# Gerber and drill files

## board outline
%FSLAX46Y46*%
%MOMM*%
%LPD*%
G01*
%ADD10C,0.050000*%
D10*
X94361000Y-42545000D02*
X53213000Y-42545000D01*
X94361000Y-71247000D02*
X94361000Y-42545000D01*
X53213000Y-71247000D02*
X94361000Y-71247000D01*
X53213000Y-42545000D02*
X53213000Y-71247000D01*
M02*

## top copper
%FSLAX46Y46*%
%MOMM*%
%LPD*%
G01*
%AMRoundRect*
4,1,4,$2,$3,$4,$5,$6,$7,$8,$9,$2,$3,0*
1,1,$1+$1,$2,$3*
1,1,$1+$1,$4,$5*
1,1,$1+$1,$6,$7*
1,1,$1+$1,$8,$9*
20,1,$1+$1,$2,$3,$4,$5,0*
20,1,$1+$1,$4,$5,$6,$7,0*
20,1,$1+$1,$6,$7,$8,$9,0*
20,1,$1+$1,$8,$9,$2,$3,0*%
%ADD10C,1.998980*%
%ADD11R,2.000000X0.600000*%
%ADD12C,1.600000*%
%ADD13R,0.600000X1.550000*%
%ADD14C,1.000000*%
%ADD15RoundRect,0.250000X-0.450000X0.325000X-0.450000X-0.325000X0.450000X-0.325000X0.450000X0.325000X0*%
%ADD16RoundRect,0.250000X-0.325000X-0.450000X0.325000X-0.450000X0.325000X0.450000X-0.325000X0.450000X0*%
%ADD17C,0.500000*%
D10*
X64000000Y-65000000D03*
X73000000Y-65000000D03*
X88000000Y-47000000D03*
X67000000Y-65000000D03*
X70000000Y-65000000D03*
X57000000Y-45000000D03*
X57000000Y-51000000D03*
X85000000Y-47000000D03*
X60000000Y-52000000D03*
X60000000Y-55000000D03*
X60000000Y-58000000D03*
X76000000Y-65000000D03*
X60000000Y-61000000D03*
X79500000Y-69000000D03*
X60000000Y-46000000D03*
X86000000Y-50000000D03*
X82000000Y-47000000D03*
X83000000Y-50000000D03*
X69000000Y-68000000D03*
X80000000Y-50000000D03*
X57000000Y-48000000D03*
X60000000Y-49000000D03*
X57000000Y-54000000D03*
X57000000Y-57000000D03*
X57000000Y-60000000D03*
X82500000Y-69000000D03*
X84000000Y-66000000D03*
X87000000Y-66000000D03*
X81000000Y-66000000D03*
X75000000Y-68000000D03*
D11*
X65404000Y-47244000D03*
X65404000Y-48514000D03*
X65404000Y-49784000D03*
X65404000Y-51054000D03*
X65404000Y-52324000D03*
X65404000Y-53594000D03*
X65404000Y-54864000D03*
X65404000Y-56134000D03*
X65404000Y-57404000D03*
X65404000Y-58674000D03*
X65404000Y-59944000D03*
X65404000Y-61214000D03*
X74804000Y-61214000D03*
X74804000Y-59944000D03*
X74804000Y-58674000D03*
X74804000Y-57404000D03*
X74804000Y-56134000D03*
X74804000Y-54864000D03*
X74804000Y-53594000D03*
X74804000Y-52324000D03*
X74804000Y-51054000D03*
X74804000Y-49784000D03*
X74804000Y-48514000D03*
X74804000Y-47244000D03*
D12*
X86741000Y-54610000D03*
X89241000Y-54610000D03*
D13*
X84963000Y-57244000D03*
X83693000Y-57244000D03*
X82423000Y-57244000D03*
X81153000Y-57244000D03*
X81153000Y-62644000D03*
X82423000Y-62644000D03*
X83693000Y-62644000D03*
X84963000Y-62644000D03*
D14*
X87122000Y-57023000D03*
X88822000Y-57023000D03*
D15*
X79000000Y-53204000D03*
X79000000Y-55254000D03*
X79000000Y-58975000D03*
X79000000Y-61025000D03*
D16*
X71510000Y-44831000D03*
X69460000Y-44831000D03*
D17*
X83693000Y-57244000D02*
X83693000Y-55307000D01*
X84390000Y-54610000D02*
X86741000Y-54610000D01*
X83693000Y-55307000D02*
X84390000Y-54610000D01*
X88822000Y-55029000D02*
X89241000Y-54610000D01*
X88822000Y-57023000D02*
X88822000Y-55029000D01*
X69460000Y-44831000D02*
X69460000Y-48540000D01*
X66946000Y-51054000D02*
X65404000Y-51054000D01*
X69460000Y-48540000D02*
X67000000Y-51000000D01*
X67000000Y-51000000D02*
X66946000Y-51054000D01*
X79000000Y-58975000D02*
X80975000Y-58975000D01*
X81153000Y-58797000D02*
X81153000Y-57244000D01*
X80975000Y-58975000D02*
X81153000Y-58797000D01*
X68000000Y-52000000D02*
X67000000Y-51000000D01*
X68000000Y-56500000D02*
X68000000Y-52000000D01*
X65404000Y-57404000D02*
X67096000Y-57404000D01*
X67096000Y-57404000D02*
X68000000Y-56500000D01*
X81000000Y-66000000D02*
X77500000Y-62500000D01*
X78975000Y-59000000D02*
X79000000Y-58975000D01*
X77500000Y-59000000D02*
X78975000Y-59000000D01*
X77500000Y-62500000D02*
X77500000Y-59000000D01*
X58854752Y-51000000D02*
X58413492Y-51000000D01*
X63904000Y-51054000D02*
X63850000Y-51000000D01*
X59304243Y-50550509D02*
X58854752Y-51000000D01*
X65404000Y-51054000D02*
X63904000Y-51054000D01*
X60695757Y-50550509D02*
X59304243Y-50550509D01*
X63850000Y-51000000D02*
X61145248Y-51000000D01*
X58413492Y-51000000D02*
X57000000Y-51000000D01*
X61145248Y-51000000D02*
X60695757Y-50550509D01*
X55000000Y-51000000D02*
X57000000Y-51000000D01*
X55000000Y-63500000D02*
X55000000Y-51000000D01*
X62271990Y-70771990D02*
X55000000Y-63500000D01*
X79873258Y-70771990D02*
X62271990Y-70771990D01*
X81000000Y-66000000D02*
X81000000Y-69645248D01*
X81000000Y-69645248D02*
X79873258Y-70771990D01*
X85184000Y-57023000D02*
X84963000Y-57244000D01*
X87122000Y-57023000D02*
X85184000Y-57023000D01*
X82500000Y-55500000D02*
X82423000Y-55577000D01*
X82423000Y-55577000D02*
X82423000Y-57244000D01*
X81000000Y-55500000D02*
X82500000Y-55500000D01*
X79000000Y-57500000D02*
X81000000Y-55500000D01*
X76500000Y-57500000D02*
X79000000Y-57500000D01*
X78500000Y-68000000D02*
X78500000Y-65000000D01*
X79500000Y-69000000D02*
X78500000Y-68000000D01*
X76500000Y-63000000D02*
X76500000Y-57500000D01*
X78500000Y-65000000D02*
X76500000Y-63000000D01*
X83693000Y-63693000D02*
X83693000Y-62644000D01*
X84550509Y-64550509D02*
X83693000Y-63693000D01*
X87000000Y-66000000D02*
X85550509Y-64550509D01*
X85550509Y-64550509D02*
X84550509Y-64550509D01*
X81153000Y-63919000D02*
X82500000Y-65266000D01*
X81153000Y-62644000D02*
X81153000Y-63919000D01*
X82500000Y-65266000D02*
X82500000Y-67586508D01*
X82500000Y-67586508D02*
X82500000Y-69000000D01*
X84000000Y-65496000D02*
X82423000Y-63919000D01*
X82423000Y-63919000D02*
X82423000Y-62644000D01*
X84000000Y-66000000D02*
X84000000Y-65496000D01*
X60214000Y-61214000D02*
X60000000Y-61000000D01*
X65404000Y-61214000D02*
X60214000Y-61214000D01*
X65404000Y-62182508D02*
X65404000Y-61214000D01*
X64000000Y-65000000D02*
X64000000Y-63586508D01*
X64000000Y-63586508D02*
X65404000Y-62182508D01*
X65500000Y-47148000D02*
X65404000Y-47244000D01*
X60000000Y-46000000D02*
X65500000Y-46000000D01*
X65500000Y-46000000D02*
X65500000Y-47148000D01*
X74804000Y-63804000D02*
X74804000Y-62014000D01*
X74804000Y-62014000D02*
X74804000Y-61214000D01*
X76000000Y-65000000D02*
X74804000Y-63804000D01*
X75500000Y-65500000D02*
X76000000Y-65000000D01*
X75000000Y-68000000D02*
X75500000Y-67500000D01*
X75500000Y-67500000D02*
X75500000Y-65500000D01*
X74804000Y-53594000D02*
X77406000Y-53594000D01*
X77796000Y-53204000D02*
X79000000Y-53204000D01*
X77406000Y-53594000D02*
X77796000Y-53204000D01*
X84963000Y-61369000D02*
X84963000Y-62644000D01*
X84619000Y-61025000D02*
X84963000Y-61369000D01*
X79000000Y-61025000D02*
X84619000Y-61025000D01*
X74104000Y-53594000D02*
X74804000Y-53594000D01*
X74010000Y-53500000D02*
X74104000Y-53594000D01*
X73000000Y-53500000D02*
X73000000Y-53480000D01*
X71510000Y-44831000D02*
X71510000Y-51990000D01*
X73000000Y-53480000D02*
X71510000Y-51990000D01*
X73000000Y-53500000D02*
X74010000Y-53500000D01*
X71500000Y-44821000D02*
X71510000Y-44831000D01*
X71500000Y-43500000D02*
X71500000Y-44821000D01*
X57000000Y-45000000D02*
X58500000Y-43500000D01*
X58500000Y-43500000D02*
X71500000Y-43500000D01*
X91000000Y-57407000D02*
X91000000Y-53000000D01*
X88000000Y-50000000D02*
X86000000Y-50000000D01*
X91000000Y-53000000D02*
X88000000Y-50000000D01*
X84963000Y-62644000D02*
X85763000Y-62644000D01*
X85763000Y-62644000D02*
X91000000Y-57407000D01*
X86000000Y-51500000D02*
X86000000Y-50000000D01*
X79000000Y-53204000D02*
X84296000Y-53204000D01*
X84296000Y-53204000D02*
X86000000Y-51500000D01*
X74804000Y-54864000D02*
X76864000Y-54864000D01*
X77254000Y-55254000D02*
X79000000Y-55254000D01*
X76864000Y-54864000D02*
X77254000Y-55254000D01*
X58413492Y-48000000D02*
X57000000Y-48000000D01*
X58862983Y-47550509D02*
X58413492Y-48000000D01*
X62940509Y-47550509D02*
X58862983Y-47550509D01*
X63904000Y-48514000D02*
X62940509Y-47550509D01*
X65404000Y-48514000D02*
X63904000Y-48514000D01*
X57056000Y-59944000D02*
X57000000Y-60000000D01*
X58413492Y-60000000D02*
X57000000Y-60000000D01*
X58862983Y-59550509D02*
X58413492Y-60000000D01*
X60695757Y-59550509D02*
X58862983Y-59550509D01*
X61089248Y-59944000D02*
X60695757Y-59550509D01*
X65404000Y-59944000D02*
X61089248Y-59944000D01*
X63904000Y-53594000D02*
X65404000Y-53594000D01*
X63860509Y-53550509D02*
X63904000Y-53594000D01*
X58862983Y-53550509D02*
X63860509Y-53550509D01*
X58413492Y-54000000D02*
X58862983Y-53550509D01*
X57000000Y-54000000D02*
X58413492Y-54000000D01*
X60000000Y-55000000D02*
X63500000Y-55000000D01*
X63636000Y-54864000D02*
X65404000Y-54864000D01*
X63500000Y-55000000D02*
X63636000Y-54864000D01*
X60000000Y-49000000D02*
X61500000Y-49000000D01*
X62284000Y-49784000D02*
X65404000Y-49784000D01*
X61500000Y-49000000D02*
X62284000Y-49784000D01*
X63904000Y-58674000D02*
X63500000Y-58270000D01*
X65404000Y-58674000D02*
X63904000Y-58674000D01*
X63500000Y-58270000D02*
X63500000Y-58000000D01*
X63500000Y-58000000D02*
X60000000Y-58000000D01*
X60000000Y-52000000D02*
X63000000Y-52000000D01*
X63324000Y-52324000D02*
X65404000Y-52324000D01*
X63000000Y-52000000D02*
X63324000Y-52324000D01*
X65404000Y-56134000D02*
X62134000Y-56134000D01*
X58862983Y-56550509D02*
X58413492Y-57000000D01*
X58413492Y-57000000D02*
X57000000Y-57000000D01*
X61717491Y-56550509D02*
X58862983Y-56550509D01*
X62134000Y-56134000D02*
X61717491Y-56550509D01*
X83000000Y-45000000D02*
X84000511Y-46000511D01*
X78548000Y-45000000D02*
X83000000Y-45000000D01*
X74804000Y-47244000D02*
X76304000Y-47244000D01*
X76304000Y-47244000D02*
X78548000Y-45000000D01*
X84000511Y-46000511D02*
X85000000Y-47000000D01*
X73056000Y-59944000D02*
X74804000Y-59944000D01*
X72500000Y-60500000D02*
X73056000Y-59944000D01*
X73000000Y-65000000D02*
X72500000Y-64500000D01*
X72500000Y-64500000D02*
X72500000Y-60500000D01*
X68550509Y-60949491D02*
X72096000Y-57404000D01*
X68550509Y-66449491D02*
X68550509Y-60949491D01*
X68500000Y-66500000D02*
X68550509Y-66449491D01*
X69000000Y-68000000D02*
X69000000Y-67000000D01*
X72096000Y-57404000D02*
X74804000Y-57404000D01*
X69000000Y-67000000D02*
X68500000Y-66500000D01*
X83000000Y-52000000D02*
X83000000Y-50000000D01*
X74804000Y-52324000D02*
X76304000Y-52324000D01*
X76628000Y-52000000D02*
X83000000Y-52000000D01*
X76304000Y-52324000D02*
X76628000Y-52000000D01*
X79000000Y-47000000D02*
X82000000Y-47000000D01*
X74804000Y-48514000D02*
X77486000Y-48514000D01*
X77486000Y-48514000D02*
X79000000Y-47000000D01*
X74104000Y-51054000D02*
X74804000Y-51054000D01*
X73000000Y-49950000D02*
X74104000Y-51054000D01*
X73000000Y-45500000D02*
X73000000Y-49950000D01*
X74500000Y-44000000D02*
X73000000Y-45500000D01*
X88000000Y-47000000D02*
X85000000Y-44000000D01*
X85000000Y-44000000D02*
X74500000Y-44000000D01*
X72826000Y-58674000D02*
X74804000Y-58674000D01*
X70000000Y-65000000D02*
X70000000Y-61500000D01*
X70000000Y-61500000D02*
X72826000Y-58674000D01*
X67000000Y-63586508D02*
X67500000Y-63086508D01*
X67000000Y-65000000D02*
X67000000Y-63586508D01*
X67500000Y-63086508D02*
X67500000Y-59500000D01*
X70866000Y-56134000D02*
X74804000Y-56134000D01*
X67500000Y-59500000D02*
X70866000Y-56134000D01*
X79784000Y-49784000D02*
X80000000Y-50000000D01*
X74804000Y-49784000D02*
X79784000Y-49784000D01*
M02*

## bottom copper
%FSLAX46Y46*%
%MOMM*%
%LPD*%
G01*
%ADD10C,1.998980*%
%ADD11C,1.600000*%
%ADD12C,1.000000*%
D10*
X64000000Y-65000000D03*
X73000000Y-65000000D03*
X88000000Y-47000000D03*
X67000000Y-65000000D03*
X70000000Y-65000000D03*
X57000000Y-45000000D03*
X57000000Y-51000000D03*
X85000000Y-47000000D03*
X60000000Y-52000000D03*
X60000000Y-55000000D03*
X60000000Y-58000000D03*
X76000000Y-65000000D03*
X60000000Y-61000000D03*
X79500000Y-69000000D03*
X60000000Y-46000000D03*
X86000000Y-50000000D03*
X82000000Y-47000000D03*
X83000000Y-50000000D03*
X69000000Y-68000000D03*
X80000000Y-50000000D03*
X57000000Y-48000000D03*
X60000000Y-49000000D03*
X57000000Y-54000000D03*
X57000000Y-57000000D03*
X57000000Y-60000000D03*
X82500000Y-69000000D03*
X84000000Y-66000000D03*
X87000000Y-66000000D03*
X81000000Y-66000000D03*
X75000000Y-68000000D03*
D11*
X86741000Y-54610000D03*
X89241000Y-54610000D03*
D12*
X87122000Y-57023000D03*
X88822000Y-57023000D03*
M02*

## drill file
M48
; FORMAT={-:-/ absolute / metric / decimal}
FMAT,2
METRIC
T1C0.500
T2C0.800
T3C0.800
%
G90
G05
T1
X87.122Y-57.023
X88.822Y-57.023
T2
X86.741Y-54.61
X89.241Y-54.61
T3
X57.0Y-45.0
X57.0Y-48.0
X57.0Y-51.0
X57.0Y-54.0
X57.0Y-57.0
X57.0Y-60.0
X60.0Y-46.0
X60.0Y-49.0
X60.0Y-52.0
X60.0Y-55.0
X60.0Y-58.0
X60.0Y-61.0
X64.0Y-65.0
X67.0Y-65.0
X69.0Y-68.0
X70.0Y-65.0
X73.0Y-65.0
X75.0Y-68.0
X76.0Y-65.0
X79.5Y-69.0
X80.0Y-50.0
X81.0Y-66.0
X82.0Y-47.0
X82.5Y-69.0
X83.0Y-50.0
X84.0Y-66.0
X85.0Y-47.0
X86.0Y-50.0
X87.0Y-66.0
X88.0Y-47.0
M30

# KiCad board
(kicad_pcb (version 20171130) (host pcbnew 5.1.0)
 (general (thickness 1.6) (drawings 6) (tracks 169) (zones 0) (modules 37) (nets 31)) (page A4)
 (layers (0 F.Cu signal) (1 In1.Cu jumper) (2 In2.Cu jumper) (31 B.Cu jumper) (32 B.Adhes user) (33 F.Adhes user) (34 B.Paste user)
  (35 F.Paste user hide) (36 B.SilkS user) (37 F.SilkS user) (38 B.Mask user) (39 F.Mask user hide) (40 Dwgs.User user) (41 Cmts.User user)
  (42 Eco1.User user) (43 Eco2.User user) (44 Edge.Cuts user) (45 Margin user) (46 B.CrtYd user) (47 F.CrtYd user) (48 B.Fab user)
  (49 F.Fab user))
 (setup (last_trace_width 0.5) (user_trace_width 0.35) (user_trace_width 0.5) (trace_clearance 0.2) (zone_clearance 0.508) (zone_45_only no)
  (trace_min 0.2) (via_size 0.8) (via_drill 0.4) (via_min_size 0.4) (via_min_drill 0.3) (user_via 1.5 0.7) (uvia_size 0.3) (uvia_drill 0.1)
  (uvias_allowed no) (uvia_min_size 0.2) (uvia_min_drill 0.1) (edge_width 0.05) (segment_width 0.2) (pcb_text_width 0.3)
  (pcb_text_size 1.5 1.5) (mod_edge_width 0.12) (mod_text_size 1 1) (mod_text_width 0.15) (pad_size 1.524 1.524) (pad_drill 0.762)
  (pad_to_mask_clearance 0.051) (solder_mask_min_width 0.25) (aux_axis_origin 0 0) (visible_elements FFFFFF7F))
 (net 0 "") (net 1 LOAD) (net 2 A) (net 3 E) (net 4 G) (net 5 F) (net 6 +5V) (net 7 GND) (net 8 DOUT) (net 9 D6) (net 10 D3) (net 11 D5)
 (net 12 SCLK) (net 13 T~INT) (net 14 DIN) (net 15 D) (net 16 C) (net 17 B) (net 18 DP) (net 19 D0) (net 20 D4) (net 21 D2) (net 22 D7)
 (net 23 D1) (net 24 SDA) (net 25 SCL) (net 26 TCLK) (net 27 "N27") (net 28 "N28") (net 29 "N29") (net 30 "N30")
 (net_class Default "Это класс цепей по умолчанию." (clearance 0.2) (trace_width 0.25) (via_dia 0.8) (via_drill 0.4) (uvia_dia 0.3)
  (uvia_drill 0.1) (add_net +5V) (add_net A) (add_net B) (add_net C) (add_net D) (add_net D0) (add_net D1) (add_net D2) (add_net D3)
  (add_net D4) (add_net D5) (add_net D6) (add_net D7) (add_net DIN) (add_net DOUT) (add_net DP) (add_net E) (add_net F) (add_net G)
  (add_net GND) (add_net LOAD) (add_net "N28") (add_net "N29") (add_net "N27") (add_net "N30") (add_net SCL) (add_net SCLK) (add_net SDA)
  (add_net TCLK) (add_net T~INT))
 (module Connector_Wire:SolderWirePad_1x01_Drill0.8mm (layer F.Cu) (at 64 65)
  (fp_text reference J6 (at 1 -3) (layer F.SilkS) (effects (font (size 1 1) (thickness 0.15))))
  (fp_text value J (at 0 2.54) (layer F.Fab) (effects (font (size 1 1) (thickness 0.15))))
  (pad 1 thru_hole circle (at 0 0) (size 1.99898 1.99898) (drill 0.8001) (layers *.Cu *.Mask) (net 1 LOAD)))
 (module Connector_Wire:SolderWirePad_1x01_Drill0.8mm (layer F.Cu) (at 73 65)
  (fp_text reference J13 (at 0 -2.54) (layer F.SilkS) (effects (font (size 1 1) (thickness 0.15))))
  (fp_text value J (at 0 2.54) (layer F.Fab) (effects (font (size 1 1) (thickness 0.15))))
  (pad 1 thru_hole circle (at 0 0) (size 1.99898 1.99898) (drill 0.8001) (layers *.Cu *.Mask) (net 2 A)))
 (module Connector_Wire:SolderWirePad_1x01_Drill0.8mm (layer F.Cu) (at 88 47)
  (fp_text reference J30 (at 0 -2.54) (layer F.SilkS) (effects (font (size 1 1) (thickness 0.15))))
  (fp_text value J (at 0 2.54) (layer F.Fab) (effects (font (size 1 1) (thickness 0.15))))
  (pad 1 thru_hole circle (at 0 0) (size 1.99898 1.99898) (drill 0.8001) (layers *.Cu *.Mask) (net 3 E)))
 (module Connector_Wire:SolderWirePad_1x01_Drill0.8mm (layer F.Cu) (at 67 65)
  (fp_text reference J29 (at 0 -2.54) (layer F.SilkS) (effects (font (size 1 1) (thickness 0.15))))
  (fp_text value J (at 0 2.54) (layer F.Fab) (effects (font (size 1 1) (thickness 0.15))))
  (pad 1 thru_hole circle (at 0 0) (size 1.99898 1.99898) (drill 0.8001) (layers *.Cu *.Mask) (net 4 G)))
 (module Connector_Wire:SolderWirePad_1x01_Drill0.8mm (layer F.Cu) (at 70 65)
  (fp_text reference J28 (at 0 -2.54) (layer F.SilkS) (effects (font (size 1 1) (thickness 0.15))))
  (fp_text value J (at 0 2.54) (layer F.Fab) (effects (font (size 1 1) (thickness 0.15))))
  (pad 1 thru_hole circle (at 0 0) (size 1.99898 1.99898) (drill 0.8001) (layers *.Cu *.Mask) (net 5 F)))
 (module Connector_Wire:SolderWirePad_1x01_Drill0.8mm (layer F.Cu) (at 57 45)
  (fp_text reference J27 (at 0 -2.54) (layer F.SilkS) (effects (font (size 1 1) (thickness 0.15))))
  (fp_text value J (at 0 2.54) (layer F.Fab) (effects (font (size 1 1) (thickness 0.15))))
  (pad 1 thru_hole circle (at 0 0) (size 1.99898 1.99898) (drill 0.8001) (layers *.Cu *.Mask) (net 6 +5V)))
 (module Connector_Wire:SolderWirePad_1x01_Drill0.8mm (layer F.Cu) (at 57 51)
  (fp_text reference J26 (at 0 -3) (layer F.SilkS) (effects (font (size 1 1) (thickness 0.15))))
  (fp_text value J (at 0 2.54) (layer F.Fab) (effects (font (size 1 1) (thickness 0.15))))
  (pad 1 thru_hole circle (at 0 0) (size 1.99898 1.99898) (drill 0.8001) (layers *.Cu *.Mask) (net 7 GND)))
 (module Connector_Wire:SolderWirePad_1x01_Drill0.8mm (layer F.Cu) (at 85 47)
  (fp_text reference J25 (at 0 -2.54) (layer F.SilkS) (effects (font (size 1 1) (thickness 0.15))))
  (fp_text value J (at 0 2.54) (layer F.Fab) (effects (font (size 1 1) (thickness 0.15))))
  (pad 1 thru_hole circle (at 0 0) (size 1.99898 1.99898) (drill 0.8001) (layers *.Cu *.Mask) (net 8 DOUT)))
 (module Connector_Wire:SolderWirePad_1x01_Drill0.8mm (layer F.Cu) (at 60 52)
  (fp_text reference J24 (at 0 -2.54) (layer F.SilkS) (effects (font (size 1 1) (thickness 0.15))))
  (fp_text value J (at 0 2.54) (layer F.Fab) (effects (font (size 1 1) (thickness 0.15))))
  (pad 1 thru_hole circle (at 0 0) (size 1.99898 1.99898) (drill 0.8001) (layers *.Cu *.Mask) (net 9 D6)))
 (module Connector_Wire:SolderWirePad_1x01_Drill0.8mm (layer F.Cu) (at 60 55)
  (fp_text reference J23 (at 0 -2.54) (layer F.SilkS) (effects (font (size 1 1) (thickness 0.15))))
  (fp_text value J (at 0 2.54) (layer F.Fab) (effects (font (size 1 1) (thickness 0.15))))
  (pad 1 thru_hole circle (at 0 0) (size 1.99898 1.99898) (drill 0.8001) (layers *.Cu *.Mask) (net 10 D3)))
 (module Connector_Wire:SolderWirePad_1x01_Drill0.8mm (layer F.Cu) (at 60 58)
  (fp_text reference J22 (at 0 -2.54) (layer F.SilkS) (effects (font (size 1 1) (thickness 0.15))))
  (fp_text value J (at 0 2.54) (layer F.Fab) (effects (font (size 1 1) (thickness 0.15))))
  (pad 1 thru_hole circle (at 0 0) (size 1.99898 1.99898) (drill 0.8001) (layers *.Cu *.Mask) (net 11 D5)))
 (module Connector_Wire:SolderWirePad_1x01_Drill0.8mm (layer F.Cu) (at 76 65)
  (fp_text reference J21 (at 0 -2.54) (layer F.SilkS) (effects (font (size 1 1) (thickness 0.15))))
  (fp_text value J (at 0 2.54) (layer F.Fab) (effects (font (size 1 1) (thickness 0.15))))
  (pad 1 thru_hole circle (at 0 0) (size 1.99898 1.99898) (drill 0.8001) (layers *.Cu *.Mask) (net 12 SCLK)))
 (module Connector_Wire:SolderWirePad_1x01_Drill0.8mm (layer F.Cu) (at 60 61)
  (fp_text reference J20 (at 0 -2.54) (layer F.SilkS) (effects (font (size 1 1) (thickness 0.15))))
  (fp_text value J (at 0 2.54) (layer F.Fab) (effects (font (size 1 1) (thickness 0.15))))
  (pad 1 thru_hole circle (at 0 0) (size 1.99898 1.99898) (drill 0.8001) (layers *.Cu *.Mask) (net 1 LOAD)))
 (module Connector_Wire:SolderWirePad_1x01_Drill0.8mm (layer F.Cu) (at 79.5 69)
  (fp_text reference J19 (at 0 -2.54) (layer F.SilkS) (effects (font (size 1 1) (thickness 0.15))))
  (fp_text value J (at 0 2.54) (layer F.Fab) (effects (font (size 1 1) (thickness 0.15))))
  (pad 1 thru_hole circle (at 0 0) (size 1.99898 1.99898) (drill 0.8001) (layers *.Cu *.Mask) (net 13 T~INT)))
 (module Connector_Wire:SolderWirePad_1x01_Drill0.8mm (layer F.Cu) (at 60 46)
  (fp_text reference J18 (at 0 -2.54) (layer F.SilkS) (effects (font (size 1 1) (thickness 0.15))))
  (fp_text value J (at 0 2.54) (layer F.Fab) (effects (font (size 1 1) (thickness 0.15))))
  (pad 1 thru_hole circle (at 0 0) (size 1.99898 1.99898) (drill 0.8001) (layers *.Cu *.Mask) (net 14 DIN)))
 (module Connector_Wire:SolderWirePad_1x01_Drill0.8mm (layer F.Cu) (at 86 50)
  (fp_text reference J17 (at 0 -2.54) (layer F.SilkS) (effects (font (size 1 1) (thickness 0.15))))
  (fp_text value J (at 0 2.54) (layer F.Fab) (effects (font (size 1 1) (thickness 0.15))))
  (pad 1 thru_hole circle (at 0 0) (size 1.99898 1.99898) (drill 0.8001) (layers *.Cu *.Mask) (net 6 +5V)))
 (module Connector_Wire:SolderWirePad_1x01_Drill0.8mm (layer F.Cu) (at 82 47)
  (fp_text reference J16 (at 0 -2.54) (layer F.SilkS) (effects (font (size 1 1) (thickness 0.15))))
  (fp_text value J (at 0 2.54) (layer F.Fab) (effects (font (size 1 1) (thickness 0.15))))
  (pad 1 thru_hole circle (at 0 0) (size 1.99898 1.99898) (drill 0.8001) (layers *.Cu *.Mask) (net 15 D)))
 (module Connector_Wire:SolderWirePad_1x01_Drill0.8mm (layer F.Cu) (at 83 50)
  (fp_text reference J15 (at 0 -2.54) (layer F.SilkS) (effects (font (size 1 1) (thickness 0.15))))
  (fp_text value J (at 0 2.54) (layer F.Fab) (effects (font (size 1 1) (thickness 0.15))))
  (pad 1 thru_hole circle (at 0 0) (size 1.99898 1.99898) (drill 0.8001) (layers *.Cu *.Mask) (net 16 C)))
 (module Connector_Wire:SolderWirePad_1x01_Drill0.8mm (layer F.Cu) (at 69 68)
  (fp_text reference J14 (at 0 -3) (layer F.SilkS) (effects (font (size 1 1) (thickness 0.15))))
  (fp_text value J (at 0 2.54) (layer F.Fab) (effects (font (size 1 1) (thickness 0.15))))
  (pad 1 thru_hole circle (at 0 0) (size 1.99898 1.99898) (drill 0.8001) (layers *.Cu *.Mask) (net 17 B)))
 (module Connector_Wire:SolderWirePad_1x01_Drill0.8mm (layer F.Cu) (at 80 50)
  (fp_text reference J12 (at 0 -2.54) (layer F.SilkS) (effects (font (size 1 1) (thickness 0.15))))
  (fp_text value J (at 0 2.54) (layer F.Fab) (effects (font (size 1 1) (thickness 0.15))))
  (pad 1 thru_hole circle (at 0 0) (size 1.99898 1.99898) (drill 0.8001) (layers *.Cu *.Mask) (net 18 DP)))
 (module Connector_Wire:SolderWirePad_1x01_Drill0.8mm (layer F.Cu) (at 57 48)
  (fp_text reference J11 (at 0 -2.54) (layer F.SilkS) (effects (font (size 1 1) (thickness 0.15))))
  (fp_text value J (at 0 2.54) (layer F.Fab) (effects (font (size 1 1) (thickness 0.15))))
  (pad 1 thru_hole circle (at 0 0) (size 1.99898 1.99898) (drill 0.8001) (layers *.Cu *.Mask) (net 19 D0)))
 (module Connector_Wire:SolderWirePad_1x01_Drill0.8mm (layer F.Cu) (at 60 49)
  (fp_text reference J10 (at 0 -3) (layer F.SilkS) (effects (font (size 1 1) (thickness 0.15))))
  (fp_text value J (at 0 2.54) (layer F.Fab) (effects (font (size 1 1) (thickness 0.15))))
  (pad 1 thru_hole circle (at 0 0) (size 1.99898 1.99898) (drill 0.8001) (layers *.Cu *.Mask) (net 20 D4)))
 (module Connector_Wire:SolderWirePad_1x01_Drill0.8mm (layer F.Cu) (at 57 54)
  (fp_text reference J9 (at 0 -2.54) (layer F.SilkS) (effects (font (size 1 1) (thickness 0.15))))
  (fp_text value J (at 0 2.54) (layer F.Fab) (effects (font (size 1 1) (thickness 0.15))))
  (pad 1 thru_hole circle (at 0 0) (size 1.99898 1.99898) (drill 0.8001) (layers *.Cu *.Mask) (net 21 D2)))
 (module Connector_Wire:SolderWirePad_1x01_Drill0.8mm (layer F.Cu) (at 57 57)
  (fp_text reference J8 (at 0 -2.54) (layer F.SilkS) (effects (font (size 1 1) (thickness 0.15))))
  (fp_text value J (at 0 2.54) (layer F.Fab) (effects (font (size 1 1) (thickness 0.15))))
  (pad 1 thru_hole circle (at 0 0) (size 1.99898 1.99898) (drill 0.8001) (layers *.Cu *.Mask) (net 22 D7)))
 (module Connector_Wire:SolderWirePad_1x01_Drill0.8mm (layer F.Cu) (at 57 60)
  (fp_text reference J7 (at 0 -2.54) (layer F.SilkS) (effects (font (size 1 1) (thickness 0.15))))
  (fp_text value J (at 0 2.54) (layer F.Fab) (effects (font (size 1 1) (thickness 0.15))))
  (pad 1 thru_hole circle (at 0 0) (size 1.99898 1.99898) (drill 0.8001) (layers *.Cu *.Mask) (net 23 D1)))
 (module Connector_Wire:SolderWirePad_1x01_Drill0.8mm (layer F.Cu) (at 82.5 69)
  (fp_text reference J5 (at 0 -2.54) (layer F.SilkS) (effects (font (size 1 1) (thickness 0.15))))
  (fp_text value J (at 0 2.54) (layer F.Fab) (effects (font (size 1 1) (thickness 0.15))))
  (pad 1 thru_hole circle (at 0 0) (size 1.99898 1.99898) (drill 0.8001) (layers *.Cu *.Mask) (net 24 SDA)))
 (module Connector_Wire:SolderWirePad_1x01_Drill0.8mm (layer F.Cu) (at 84 66)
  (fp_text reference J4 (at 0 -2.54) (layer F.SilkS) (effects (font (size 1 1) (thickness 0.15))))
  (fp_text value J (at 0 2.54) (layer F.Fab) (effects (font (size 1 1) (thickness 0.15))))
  (pad 1 thru_hole circle (at 0 0) (size 1.99898 1.99898) (drill 0.8001) (layers *.Cu *.Mask) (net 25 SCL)))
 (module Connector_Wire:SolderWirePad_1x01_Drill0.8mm (layer F.Cu) (at 87 66)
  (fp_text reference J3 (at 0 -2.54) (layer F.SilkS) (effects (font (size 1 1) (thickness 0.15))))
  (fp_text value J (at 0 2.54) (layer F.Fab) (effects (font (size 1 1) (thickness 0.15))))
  (pad 1 thru_hole circle (at 0 0) (size 1.99898 1.99898) (drill 0.8001) (layers *.Cu *.Mask) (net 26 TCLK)))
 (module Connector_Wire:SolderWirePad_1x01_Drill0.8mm (layer F.Cu) (at 81 66)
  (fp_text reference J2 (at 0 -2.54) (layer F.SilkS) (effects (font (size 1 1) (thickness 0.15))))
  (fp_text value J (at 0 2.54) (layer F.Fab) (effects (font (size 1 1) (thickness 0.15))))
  (pad 1 thru_hole circle (at 0 0) (size 1.99898 1.99898) (drill 0.8001) (layers *.Cu *.Mask) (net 7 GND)))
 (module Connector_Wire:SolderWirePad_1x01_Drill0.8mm (layer F.Cu) (at 75 68)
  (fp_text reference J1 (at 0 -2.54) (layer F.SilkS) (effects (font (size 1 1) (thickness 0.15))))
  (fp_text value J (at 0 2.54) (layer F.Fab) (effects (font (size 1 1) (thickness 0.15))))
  (pad 1 thru_hole circle (at 0 0) (size 1.99898 1.99898) (drill 0.8001) (layers *.Cu *.Mask) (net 12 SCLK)))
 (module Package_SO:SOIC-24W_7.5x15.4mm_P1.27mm (layer F.Cu) (at 70.104 54.229)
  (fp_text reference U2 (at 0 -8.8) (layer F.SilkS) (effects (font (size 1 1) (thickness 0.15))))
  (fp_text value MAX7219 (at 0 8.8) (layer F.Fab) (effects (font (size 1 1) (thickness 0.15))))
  (pad 1 smd rect (at -4.7 -6.985) (size 2 0.6) (layers F.Cu F.Paste F.Mask) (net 14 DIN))
  (pad 2 smd rect (at -4.7 -5.715) (size 2 0.6) (layers F.Cu F.Paste F.Mask) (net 19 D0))
  (pad 3 smd rect (at -4.7 -4.445) (size 2 0.6) (layers F.Cu F.Paste F.Mask) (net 20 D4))
  (pad 4 smd rect (at -4.7 -3.175) (size 2 0.6) (layers F.Cu F.Paste F.Mask) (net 7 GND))
  (pad 5 smd rect (at -4.7 -1.905) (size 2 0.6) (layers F.Cu F.Paste F.Mask) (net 9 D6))
  (pad 6 smd rect (at -4.7 -0.635) (size 2 0.6) (layers F.Cu F.Paste F.Mask) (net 21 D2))
  (pad 7 smd rect (at -4.7 0.635) (size 2 0.6) (layers F.Cu F.Paste F.Mask) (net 10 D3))
  (pad 8 smd rect (at -4.7 1.905) (size 2 0.6) (layers F.Cu F.Paste F.Mask) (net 22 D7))
  (pad 9 smd rect (at -4.7 3.175) (size 2 0.6) (layers F.Cu F.Paste F.Mask) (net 7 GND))
  (pad 10 smd rect (at -4.7 4.445) (size 2 0.6) (layers F.Cu F.Paste F.Mask) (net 11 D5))
  (pad 11 smd rect (at -4.7 5.715) (size 2 0.6) (layers F.Cu F.Paste F.Mask) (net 23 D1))
  (pad 12 smd rect (at -4.7 6.985) (size 2 0.6) (layers F.Cu F.Paste F.Mask) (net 1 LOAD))
  (pad 13 smd rect (at 4.7 6.985) (size 2 0.6) (layers F.Cu F.Paste F.Mask) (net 12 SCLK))
  (pad 14 smd rect (at 4.7 5.715) (size 2 0.6) (layers F.Cu F.Paste F.Mask) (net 2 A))
  (pad 15 smd rect (at 4.7 4.445) (size 2 0.6) (layers F.Cu F.Paste F.Mask) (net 5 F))
  (pad 16 smd rect (at 4.7 3.175) (size 2 0.6) (layers F.Cu F.Paste F.Mask) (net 17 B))
  (pad 17 smd rect (at 4.7 1.905) (size 2 0.6) (layers F.Cu F.Paste F.Mask) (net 4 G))
  (pad 18 smd rect (at 4.7 0.635) (size 2 0.6) (layers F.Cu F.Paste F.Mask) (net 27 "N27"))
  (pad 19 smd rect (at 4.7 -0.635) (size 2 0.6) (layers F.Cu F.Paste F.Mask) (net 6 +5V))
  (pad 20 smd rect (at 4.7 -1.905) (size 2 0.6) (layers F.Cu F.Paste F.Mask) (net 16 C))
  (pad 21 smd rect (at 4.7 -3.175) (size 2 0.6) (layers F.Cu F.Paste F.Mask) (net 3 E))
  (pad 22 smd rect (at 4.7 -4.445) (size 2 0.6) (layers F.Cu F.Paste F.Mask) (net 18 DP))
  (pad 23 smd rect (at 4.7 -5.715) (size 2 0.6) (layers F.Cu F.Paste F.Mask) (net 15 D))
  (pad 24 smd rect (at 4.7 -6.985) (size 2 0.6) (layers F.Cu F.Paste F.Mask) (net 8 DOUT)))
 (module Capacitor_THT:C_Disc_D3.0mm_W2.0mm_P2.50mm (layer B.Cu) (at 86.741 54.61)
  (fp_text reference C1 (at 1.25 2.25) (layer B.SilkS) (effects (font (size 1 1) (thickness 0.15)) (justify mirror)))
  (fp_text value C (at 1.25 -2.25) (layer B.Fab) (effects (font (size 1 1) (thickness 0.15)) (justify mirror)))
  (pad 1 thru_hole circle (at 0 0) (size 1.6 1.6) (drill 0.8) (layers *.Cu *.Mask) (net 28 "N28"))
  (pad 2 thru_hole circle (at 2.5 0) (size 1.6 1.6) (drill 0.8) (layers *.Cu *.Mask) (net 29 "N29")))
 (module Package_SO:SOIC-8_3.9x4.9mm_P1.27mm (layer F.Cu) (at 83.058 59.944 270)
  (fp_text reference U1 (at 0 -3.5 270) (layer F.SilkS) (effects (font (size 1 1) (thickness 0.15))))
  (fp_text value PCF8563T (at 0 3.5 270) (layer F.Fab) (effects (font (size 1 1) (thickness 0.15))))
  (pad 1 smd rect (at -2.7 -1.905 270) (size 1.55 0.6) (layers F.Cu F.Paste F.Mask) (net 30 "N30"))
  (pad 2 smd rect (at -2.7 -0.635 270) (size 1.55 0.6) (layers F.Cu F.Paste F.Mask) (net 28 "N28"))
  (pad 3 smd rect (at -2.7 0.635 270) (size 1.55 0.6) (layers F.Cu F.Paste F.Mask) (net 13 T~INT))
  (pad 4 smd rect (at -2.7 1.905 270) (size 1.55 0.6) (layers F.Cu F.Paste F.Mask) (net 7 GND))
  (pad 5 smd rect (at 2.7 1.905 270) (size 1.55 0.6) (layers F.Cu F.Paste F.Mask) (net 24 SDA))
  (pad 6 smd rect (at 2.7 0.635 270) (size 1.55 0.6) (layers F.Cu F.Paste F.Mask) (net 25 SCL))
  (pad 7 smd rect (at 2.7 -0.635 270) (size 1.55 0.6) (layers F.Cu F.Paste F.Mask) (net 26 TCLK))
  (pad 8 smd rect (at 2.7 -1.905 270) (size 1.55 0.6) (layers F.Cu F.Paste F.Mask) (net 6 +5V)))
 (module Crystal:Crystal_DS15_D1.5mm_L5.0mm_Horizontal (layer F.Cu) (at 87.122 57.023)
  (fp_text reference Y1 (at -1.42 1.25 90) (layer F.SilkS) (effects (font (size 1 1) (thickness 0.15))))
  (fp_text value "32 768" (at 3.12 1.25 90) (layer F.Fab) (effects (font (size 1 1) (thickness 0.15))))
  (pad 1 thru_hole circle (at 0 0) (size 1 1) (drill 0.5) (layers *.Cu *.Mask) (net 30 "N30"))
  (pad 2 thru_hole circle (at 1.7 0) (size 1 1) (drill 0.5) (layers *.Cu *.Mask) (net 29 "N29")))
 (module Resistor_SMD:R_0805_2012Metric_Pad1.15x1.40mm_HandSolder (layer F.Cu) (at 79 54.229 270)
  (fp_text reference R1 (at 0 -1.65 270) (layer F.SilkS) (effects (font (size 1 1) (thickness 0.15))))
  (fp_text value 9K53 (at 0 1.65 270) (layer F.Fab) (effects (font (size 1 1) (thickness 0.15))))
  (pad 1 smd roundrect (at -1.025 0 270) (size 1.15 1.4) (layers F.Cu F.Paste F.Mask) (roundrect_rratio 0.217391) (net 6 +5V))
  (pad 2 smd roundrect (at 1.025 0 270) (size 1.15 1.4) (layers F.Cu F.Paste F.Mask) (roundrect_rratio 0.217391) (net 27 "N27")))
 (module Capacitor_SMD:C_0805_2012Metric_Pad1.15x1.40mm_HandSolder (layer F.Cu) (at 79 60 270)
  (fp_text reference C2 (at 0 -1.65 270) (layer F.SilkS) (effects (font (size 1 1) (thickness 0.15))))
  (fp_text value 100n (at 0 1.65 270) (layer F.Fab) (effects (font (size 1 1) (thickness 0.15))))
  (pad 1 smd roundrect (at -1.025 0 270) (size 1.15 1.4) (layers F.Cu F.Paste F.Mask) (roundrect_rratio 0.217391) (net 7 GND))
  (pad 2 smd roundrect (at 1.025 0 270) (size 1.15 1.4) (layers F.Cu F.Paste F.Mask) (roundrect_rratio 0.217391) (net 6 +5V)))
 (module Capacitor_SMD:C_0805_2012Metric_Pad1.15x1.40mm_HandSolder (layer F.Cu) (at 70.485 44.831)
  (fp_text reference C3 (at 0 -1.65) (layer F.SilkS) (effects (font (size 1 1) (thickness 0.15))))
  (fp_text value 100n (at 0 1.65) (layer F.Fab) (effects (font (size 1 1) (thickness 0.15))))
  (pad 2 smd roundrect (at 1.025 0) (size 1.15 1.4) (layers F.Cu F.Paste F.Mask) (roundrect_rratio 0.217391) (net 6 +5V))
  (pad 1 smd roundrect (at -1.025 0) (size 1.15 1.4) (layers F.Cu F.Paste F.Mask) (roundrect_rratio 0.217391) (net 7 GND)))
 (gr_line (start 94.361 42.545) (end 53.213 42.545) (layer Edge.Cuts) (width 0.05))
 (gr_line (start 94.361 71.247) (end 94.361 42.545) (layer Edge.Cuts) (width 0.05))
 (gr_line (start 53.213 71.247) (end 94.361 71.247) (layer Edge.Cuts) (width 0.05))
 (gr_line (start 53.213 42.545) (end 53.213 71.247) (layer Edge.Cuts) (width 0.05))
 (segment (start 83.693 57.244) (end 83.693 55.307) (width 0.5) (layer F.Cu) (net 28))
 (segment (start 84.39 54.61) (end 86.741 54.61) (width 0.5) (layer F.Cu) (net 28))
 (segment (start 83.693 55.307) (end 84.39 54.61) (width 0.5) (layer F.Cu) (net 28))
 (segment (start 88.822 55.029) (end 89.241 54.61) (width 0.5) (layer F.Cu) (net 29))
 (segment (start 88.822 57.023) (end 88.822 55.029) (width 0.5) (layer F.Cu) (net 29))
 (segment (start 69.46 44.831) (end 69.46 48.54) (width 0.5) (layer F.Cu) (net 7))
 (segment (start 66.946 51.054) (end 65.404 51.054) (width 0.5) (layer F.Cu) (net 7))
 (segment (start 69.46 48.54) (end 67 51) (width 0.5) (layer F.Cu) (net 7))
 (segment (start 67 51) (end 66.946 51.054) (width 0.5) (layer F.Cu) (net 7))
 (segment (start 79 58.975) (end 80.975 58.975) (width 0.5) (layer F.Cu) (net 7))
 (segment (start 81.153 58.797) (end 81.153 57.244) (width 0.5) (layer F.Cu) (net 7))
 (segment (start 80.975 58.975) (end 81.153 58.797) (width 0.5) (layer F.Cu) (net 7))
 (segment (start 68 52) (end 67 51) (width 0.5) (layer F.Cu) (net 7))
 (segment (start 68 56.5) (end 68 52) (width 0.5) (layer F.Cu) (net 7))
 (segment (start 65.404 57.404) (end 67.096 57.404) (width 0.5) (layer F.Cu) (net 7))
 (segment (start 67.096 57.404) (end 68 56.5) (width 0.5) (layer F.Cu) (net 7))
 (segment (start 81 66) (end 77.5 62.5) (width 0.5) (layer F.Cu) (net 7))
 (segment (start 78.975 59) (end 79 58.975) (width 0.5) (layer F.Cu) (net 7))
 (segment (start 77.5 59) (end 78.975 59) (width 0.5) (layer F.Cu) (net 7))
 (segment (start 77.5 62.5) (end 77.5 59) (width 0.5) (layer F.Cu) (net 7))
 (segment (start 58.854752 51) (end 58.413492 51) (width 0.5) (layer F.Cu) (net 7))
 (segment (start 63.904 51.054) (end 63.85 51) (width 0.5) (layer F.Cu) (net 7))
 (segment (start 59.304243 50.550509) (end 58.854752 51) (width 0.5) (layer F.Cu) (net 7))
 (segment (start 65.404 51.054) (end 63.904 51.054) (width 0.5) (layer F.Cu) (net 7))
 (segment (start 60.695757 50.550509) (end 59.304243 50.550509) (width 0.5) (layer F.Cu) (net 7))
 (segment (start 63.85 51) (end 61.145248 51) (width 0.5) (layer F.Cu) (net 7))
 (segment (start 58.413492 51) (end 57 51) (width 0.5) (layer F.Cu) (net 7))
 (segment (start 61.145248 51) (end 60.695757 50.550509) (width 0.5) (layer F.Cu) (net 7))
 (segment (start 55 51) (end 57 51) (width 0.5) (layer F.Cu) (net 7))
 (segment (start 55 63.5) (end 55 51) (width 0.5) (layer F.Cu) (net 7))
 (segment (start 62.27199 70.77199) (end 55 63.5) (width 0.5) (layer F.Cu) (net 7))
 (segment (start 79.873258 70.77199) (end 62.27199 70.77199) (width 0.5) (layer F.Cu) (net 7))
 (segment (start 81 66) (end 81 69.645248) (width 0.5) (layer F.Cu) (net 7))
 (segment (start 81 69.645248) (end 79.873258 70.77199) (width 0.5) (layer F.Cu) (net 7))
 (segment (start 85.184 57.023) (end 84.963 57.244) (width 0.5) (layer F.Cu) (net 30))
 (segment (start 87.122 57.023) (end 85.184 57.023) (width 0.5) (layer F.Cu) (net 30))
 (segment (start 82.5 55.5) (end 82.423 55.577) (width 0.5) (layer F.Cu) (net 13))
 (segment (start 82.423 55.577) (end 82.423 57.244) (width 0.5) (layer F.Cu) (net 13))
 (segment (start 81 55.5) (end 82.5 55.5) (width 0.5) (layer F.Cu) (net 13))
 (segment (start 79 57.5) (end 81 55.5) (width 0.5) (layer F.Cu) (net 13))
 (segment (start 76.5 57.5) (end 79 57.5) (width 0.5) (layer F.Cu) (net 13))
 (segment (start 78.5 68) (end 78.5 65) (width 0.5) (layer F.Cu) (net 13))
 (segment (start 79.5 69) (end 78.5 68) (width 0.5) (layer F.Cu) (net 13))
 (segment (start 76.5 63) (end 76.5 57.5) (width 0.5) (layer F.Cu) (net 13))
 (segment (start 78.5 65) (end 76.5 63) (width 0.5) (layer F.Cu) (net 13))
 (segment (start 83.693 63.693) (end 83.693 62.644) (width 0.5) (layer F.Cu) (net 26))
 (segment (start 84.550509 64.550509) (end 83.693 63.693) (width 0.5) (layer F.Cu) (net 26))
 (segment (start 87 66) (end 85.550509 64.550509) (width 0.5) (layer F.Cu) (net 26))
 (segment (start 85.550509 64.550509) (end 84.550509 64.550509) (width 0.5) (layer F.Cu) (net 26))
 (segment (start 81.153 63.919) (end 82.5 65.266) (width 0.5) (layer F.Cu) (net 24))
 (segment (start 81.153 62.644) (end 81.153 63.919) (width 0.5) (layer F.Cu) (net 24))
 (segment (start 82.5 65.266) (end 82.5 67.586508) (width 0.5) (layer F.Cu) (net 24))
 (segment (start 82.5 67.586508) (end 82.5 69) (width 0.5) (layer F.Cu) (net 24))
 (segment (start 84 65.496) (end 82.423 63.919) (width 0.5) (layer F.Cu) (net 25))
 (segment (start 82.423 63.919) (end 82.423 62.644) (width 0.5) (layer F.Cu) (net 25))
 (segment (start 84 66) (end 84 65.496) (width 0.5) (layer F.Cu) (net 25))
 (segment (start 60.214 61.214) (end 60 61) (width 0.5) (layer F.Cu) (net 1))
 (segment (start 65.404 61.214) (end 60.214 61.214) (width 0.5) (layer F.Cu) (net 1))
 (segment (start 65.404 62.182508) (end 65.404 61.214) (width 0.5) (layer F.Cu) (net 1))
 (segment (start 64 65) (end 64 63.586508) (width 0.5) (layer F.Cu) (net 1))
 (segment (start 64 63.586508) (end 65.404 62.182508) (width 0.5) (layer F.Cu) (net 1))
 (segment (start 65.5 47.148) (end 65.404 47.244) (width 0.5) (layer F.Cu) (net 14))
 (segment (start 60 46) (end 65.5 46) (width 0.5) (layer F.Cu) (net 14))
 (segment (start 65.5 46) (end 65.5 47.148) (width 0.5) (layer F.Cu) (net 14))
 (segment (start 74.804 63.804) (end 74.804 62.014) (width 0.5) (layer F.Cu) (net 12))
 (segment (start 74.804 62.014) (end 74.804 61.214) (width 0.5) (layer F.Cu) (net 12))
 (segment (start 76 65) (end 74.804 63.804) (width 0.5) (layer F.Cu) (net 12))
 (segment (start 75.5 65.5) (end 76 65) (width 0.5) (layer F.Cu) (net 12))
 (segment (start 75 68) (end 75.5 67.5) (width 0.5) (layer F.Cu) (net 12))
 (segment (start 75.5 67.5) (end 75.5 65.5) (width 0.5) (layer F.Cu) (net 12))
 (segment (start 74.804 53.594) (end 77.406 53.594) (width 0.5) (layer F.Cu) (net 6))
 (segment (start 77.796 53.204) (end 79 53.204) (width 0.5) (layer F.Cu) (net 6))
 (segment (start 77.406 53.594) (end 77.796 53.204) (width 0.5) (layer F.Cu) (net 6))
 (segment (start 84.963 61.369) (end 84.963 62.644) (width 0.5) (layer F.Cu) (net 6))
 (segment (start 84.619 61.025) (end 84.963 61.369) (width 0.5) (layer F.Cu) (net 6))
 (segment (start 79 61.025) (end 84.619 61.025) (width 0.5) (layer F.Cu) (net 6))
 (segment (start 74.104 53.594) (end 74.804 53.594) (width 0.5) (layer F.Cu) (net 6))
 (segment (start 74.01 53.5) (end 74.104 53.594) (width 0.5) (layer F.Cu) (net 6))
 (segment (start 73 53.5) (end 73 53.48) (width 0.5) (layer F.Cu) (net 6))
 (segment (start 71.51 44.831) (end 71.51 51.99) (width 0.5) (layer F.Cu) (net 6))
 (segment (start 73 53.48) (end 71.51 51.99) (width 0.5) (layer F.Cu) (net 6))
 (segment (start 73 53.5) (end 74.01 53.5) (width 0.5) (layer F.Cu) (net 6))
 (segment (start 71.5 44.821) (end 71.51 44.831) (width 0.5) (layer F.Cu) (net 6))
 (segment (start 71.5 43.5) (end 71.5 44.821) (width 0.5) (layer F.Cu) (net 6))
 (segment (start 57 45) (end 58.5 43.5) (width 0.5) (layer F.Cu) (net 6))
 (segment (start 58.5 43.5) (end 71.5 43.5) (width 0.5) (layer F.Cu) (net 6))
 (segment (start 91 57.407) (end 91 53) (width 0.5) (layer F.Cu) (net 6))
 (segment (start 88 50) (end 86 50) (width 0.5) (layer F.Cu) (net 6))
 (segment (start 91 53) (end 88 50) (width 0.5) (layer F.Cu) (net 6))
 (segment (start 84.963 62.644) (end 85.763 62.644) (width 0.5) (layer F.Cu) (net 6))
 (segment (start 85.763 62.644) (end 91 57.407) (width 0.5) (layer F.Cu) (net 6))
 (segment (start 86 51.5) (end 86 50) (width 0.5) (layer F.Cu) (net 6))
 (segment (start 79 53.204) (end 84.296 53.204) (width 0.5) (layer F.Cu) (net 6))
 (segment (start 84.296 53.204) (end 86 51.5) (width 0.5) (layer F.Cu) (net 6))
 (segment (start 74.804 54.864) (end 76.864 54.864) (width 0.5) (layer F.Cu) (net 27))
 (segment (start 77.254 55.254) (end 79 55.254) (width 0.5) (layer F.Cu) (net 27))
 (segment (start 76.864 54.864) (end 77.254 55.254) (width 0.5) (layer F.Cu) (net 27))
 (segment (start 58.413492 48) (end 57 48) (width 0.5) (layer F.Cu) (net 19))
 (segment (start 58.862983 47.550509) (end 58.413492 48) (width 0.5) (layer F.Cu) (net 19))
 (segment (start 62.940509 47.550509) (end 58.862983 47.550509) (width 0.5) (layer F.Cu) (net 19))
 (segment (start 63.904 48.514) (end 62.940509 47.550509) (width 0.5) (layer F.Cu) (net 19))
 (segment (start 65.404 48.514) (end 63.904 48.514) (width 0.5) (layer F.Cu) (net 19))
 (segment (start 57.056 59.944) (end 57 60) (width 0.5) (layer F.Cu) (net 23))
 (segment (start 58.413492 60) (end 57 60) (width 0.5) (layer F.Cu) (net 23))
 (segment (start 58.862983 59.550509) (end 58.413492 60) (width 0.5) (layer F.Cu) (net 23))
 (segment (start 60.695757 59.550509) (end 58.862983 59.550509) (width 0.5) (layer F.Cu) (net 23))
 (segment (start 61.089248 59.944) (end 60.695757 59.550509) (width 0.5) (layer F.Cu) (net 23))
 (segment (start 65.404 59.944) (end 61.089248 59.944) (width 0.5) (layer F.Cu) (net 23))
 (segment (start 63.904 53.594) (end 65.404 53.594) (width 0.5) (layer F.Cu) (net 21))
 (segment (start 63.860509 53.550509) (end 63.904 53.594) (width 0.5) (layer F.Cu) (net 21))
 (segment (start 58.862983 53.550509) (end 63.860509 53.550509) (width 0.5) (layer F.Cu) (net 21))
 (segment (start 58.413492 54) (end 58.862983 53.550509) (width 0.5) (layer F.Cu) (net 21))
 (segment (start 57 54) (end 58.413492 54) (width 0.5) (layer F.Cu) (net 21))
 (segment (start 60 55) (end 63.5 55) (width 0.5) (layer F.Cu) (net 10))
 (segment (start 63.636 54.864) (end 65.404 54.864) (width 0.5) (layer F.Cu) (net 10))
 (segment (start 63.5 55) (end 63.636 54.864) (width 0.5) (layer F.Cu) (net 10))
 (segment (start 60 49) (end 61.5 49) (width 0.5) (layer F.Cu) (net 20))
 (segment (start 62.284 49.784) (end 65.404 49.784) (width 0.5) (layer F.Cu) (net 20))
 (segment (start 61.5 49) (end 62.284 49.784) (width 0.5) (layer F.Cu) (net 20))
 (segment (start 63.904 58.674) (end 63.5 58.27) (width 0.5) (layer F.Cu) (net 11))
 (segment (start 65.404 58.674) (end 63.904 58.674) (width 0.5) (layer F.Cu) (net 11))
 (segment (start 63.5 58.27) (end 63.5 58) (width 0.5) (layer F.Cu) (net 11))
 (segment (start 63.5 58) (end 60 58) (width 0.5) (layer F.Cu) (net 11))
 (segment (start 60 52) (end 63 52) (width 0.5) (layer F.Cu) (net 9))
 (segment (start 63.324 52.324) (end 65.404 52.324) (width 0.5) (layer F.Cu) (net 9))
 (segment (start 63 52) (end 63.324 52.324) (width 0.5) (layer F.Cu) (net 9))
 (segment (start 65.404 56.134) (end 62.134 56.134) (width 0.5) (layer F.Cu) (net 22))
 (segment (start 58.862983 56.550509) (end 58.413492 57) (width 0.5) (layer F.Cu) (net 22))
 (segment (start 58.413492 57) (end 57 57) (width 0.5) (layer F.Cu) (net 22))
 (segment (start 61.717491 56.550509) (end 58.862983 56.550509) (width 0.5) (layer F.Cu) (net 22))
 (segment (start 62.134 56.134) (end 61.717491 56.550509) (width 0.5) (layer F.Cu) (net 22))
 (segment (start 83 45) (end 84.000511 46.000511) (width 0.5) (layer F.Cu) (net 8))
 (segment (start 78.548 45) (end 83 45) (width 0.5) (layer F.Cu) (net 8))
 (segment (start 74.804 47.244) (end 76.304 47.244) (width 0.5) (layer F.Cu) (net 8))
 (segment (start 76.304 47.244) (end 78.548 45) (width 0.5) (layer F.Cu) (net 8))
 (segment (start 84.000511 46.000511) (end 85 47) (width 0.5) (layer F.Cu) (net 8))
 (segment (start 73.056 59.944) (end 74.804 59.944) (width 0.5) (layer F.Cu) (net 2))
 (segment (start 72.5 60.5) (end 73.056 59.944) (width 0.5) (layer F.Cu) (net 2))
 (segment (start 73 65) (end 72.5 64.5) (width 0.5) (layer F.Cu) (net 2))
 (segment (start 72.5 64.5) (end 72.5 60.5) (width 0.5) (layer F.Cu) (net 2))
 (segment (start 68.550509 60.949491) (end 72.096 57.404) (width 0.5) (layer F.Cu) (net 17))
 (segment (start 68.550509 66.449491) (end 68.550509 60.949491) (width 0.5) (layer F.Cu) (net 17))
 (segment (start 68.5 66.5) (end 68.550509 66.449491) (width 0.5) (layer F.Cu) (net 17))
 (segment (start 69 68) (end 69 67) (width 0.5) (layer F.Cu) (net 17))
 (segment (start 72.096 57.404) (end 74.804 57.404) (width 0.5) (layer F.Cu) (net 17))
 (segment (start 69 67) (end 68.5 66.5) (width 0.5) (layer F.Cu) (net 17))
 (segment (start 83 52) (end 83 50) (width 0.5) (layer F.Cu) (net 16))
 (segment (start 74.804 52.324) (end 76.304 52.324) (width 0.5) (layer F.Cu) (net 16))
 (segment (start 76.628 52) (end 83 52) (width 0.5) (layer F.Cu) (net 16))
 (segment (start 76.304 52.324) (end 76.628 52) (width 0.5) (layer F.Cu) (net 16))
 (segment (start 79 47) (end 82 47) (width 0.5) (layer F.Cu) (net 15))
 (segment (start 74.804 48.514) (end 77.486 48.514) (width 0.5) (layer F.Cu) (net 15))
 (segment (start 77.486 48.514) (end 79 47) (width 0.5) (layer F.Cu) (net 15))
 (segment (start 74.104 51.054) (end 74.804 51.054) (width 0.5) (layer F.Cu) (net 3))
 (segment (start 73 49.95) (end 74.104 51.054) (width 0.5) (layer F.Cu) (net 3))
 (segment (start 73 45.5) (end 73 49.95) (width 0.5) (layer F.Cu) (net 3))
 (segment (start 74.5 44) (end 73 45.5) (width 0.5) (layer F.Cu) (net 3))
 (segment (start 88 47) (end 85 44) (width 0.5) (layer F.Cu) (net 3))
 (segment (start 85 44) (end 74.5 44) (width 0.5) (layer F.Cu) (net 3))
 (segment (start 72.826 58.674) (end 74.804 58.674) (width 0.5) (layer F.Cu) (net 5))
 (segment (start 70 65) (end 70 61.5) (width 0.5) (layer F.Cu) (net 5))
 (segment (start 70 61.5) (end 72.826 58.674) (width 0.5) (layer F.Cu) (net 5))
 (segment (start 67 63.586508) (end 67.5 63.086508) (width 0.5) (layer F.Cu) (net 4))
 (segment (start 67 65) (end 67 63.586508) (width 0.5) (layer F.Cu) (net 4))
 (segment (start 67.5 63.086508) (end 67.5 59.5) (width 0.5) (layer F.Cu) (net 4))
 (segment (start 70.866 56.134) (end 74.804 56.134) (width 0.5) (layer F.Cu) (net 4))
 (segment (start 67.5 59.5) (end 70.866 56.134) (width 0.5) (layer F.Cu) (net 4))
 (segment (start 79.784 49.784) (end 80 50) (width 0.5) (layer F.Cu) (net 18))
 (segment (start 74.804 49.784) (end 79.784 49.784) (width 0.5) (layer F.Cu) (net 18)))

